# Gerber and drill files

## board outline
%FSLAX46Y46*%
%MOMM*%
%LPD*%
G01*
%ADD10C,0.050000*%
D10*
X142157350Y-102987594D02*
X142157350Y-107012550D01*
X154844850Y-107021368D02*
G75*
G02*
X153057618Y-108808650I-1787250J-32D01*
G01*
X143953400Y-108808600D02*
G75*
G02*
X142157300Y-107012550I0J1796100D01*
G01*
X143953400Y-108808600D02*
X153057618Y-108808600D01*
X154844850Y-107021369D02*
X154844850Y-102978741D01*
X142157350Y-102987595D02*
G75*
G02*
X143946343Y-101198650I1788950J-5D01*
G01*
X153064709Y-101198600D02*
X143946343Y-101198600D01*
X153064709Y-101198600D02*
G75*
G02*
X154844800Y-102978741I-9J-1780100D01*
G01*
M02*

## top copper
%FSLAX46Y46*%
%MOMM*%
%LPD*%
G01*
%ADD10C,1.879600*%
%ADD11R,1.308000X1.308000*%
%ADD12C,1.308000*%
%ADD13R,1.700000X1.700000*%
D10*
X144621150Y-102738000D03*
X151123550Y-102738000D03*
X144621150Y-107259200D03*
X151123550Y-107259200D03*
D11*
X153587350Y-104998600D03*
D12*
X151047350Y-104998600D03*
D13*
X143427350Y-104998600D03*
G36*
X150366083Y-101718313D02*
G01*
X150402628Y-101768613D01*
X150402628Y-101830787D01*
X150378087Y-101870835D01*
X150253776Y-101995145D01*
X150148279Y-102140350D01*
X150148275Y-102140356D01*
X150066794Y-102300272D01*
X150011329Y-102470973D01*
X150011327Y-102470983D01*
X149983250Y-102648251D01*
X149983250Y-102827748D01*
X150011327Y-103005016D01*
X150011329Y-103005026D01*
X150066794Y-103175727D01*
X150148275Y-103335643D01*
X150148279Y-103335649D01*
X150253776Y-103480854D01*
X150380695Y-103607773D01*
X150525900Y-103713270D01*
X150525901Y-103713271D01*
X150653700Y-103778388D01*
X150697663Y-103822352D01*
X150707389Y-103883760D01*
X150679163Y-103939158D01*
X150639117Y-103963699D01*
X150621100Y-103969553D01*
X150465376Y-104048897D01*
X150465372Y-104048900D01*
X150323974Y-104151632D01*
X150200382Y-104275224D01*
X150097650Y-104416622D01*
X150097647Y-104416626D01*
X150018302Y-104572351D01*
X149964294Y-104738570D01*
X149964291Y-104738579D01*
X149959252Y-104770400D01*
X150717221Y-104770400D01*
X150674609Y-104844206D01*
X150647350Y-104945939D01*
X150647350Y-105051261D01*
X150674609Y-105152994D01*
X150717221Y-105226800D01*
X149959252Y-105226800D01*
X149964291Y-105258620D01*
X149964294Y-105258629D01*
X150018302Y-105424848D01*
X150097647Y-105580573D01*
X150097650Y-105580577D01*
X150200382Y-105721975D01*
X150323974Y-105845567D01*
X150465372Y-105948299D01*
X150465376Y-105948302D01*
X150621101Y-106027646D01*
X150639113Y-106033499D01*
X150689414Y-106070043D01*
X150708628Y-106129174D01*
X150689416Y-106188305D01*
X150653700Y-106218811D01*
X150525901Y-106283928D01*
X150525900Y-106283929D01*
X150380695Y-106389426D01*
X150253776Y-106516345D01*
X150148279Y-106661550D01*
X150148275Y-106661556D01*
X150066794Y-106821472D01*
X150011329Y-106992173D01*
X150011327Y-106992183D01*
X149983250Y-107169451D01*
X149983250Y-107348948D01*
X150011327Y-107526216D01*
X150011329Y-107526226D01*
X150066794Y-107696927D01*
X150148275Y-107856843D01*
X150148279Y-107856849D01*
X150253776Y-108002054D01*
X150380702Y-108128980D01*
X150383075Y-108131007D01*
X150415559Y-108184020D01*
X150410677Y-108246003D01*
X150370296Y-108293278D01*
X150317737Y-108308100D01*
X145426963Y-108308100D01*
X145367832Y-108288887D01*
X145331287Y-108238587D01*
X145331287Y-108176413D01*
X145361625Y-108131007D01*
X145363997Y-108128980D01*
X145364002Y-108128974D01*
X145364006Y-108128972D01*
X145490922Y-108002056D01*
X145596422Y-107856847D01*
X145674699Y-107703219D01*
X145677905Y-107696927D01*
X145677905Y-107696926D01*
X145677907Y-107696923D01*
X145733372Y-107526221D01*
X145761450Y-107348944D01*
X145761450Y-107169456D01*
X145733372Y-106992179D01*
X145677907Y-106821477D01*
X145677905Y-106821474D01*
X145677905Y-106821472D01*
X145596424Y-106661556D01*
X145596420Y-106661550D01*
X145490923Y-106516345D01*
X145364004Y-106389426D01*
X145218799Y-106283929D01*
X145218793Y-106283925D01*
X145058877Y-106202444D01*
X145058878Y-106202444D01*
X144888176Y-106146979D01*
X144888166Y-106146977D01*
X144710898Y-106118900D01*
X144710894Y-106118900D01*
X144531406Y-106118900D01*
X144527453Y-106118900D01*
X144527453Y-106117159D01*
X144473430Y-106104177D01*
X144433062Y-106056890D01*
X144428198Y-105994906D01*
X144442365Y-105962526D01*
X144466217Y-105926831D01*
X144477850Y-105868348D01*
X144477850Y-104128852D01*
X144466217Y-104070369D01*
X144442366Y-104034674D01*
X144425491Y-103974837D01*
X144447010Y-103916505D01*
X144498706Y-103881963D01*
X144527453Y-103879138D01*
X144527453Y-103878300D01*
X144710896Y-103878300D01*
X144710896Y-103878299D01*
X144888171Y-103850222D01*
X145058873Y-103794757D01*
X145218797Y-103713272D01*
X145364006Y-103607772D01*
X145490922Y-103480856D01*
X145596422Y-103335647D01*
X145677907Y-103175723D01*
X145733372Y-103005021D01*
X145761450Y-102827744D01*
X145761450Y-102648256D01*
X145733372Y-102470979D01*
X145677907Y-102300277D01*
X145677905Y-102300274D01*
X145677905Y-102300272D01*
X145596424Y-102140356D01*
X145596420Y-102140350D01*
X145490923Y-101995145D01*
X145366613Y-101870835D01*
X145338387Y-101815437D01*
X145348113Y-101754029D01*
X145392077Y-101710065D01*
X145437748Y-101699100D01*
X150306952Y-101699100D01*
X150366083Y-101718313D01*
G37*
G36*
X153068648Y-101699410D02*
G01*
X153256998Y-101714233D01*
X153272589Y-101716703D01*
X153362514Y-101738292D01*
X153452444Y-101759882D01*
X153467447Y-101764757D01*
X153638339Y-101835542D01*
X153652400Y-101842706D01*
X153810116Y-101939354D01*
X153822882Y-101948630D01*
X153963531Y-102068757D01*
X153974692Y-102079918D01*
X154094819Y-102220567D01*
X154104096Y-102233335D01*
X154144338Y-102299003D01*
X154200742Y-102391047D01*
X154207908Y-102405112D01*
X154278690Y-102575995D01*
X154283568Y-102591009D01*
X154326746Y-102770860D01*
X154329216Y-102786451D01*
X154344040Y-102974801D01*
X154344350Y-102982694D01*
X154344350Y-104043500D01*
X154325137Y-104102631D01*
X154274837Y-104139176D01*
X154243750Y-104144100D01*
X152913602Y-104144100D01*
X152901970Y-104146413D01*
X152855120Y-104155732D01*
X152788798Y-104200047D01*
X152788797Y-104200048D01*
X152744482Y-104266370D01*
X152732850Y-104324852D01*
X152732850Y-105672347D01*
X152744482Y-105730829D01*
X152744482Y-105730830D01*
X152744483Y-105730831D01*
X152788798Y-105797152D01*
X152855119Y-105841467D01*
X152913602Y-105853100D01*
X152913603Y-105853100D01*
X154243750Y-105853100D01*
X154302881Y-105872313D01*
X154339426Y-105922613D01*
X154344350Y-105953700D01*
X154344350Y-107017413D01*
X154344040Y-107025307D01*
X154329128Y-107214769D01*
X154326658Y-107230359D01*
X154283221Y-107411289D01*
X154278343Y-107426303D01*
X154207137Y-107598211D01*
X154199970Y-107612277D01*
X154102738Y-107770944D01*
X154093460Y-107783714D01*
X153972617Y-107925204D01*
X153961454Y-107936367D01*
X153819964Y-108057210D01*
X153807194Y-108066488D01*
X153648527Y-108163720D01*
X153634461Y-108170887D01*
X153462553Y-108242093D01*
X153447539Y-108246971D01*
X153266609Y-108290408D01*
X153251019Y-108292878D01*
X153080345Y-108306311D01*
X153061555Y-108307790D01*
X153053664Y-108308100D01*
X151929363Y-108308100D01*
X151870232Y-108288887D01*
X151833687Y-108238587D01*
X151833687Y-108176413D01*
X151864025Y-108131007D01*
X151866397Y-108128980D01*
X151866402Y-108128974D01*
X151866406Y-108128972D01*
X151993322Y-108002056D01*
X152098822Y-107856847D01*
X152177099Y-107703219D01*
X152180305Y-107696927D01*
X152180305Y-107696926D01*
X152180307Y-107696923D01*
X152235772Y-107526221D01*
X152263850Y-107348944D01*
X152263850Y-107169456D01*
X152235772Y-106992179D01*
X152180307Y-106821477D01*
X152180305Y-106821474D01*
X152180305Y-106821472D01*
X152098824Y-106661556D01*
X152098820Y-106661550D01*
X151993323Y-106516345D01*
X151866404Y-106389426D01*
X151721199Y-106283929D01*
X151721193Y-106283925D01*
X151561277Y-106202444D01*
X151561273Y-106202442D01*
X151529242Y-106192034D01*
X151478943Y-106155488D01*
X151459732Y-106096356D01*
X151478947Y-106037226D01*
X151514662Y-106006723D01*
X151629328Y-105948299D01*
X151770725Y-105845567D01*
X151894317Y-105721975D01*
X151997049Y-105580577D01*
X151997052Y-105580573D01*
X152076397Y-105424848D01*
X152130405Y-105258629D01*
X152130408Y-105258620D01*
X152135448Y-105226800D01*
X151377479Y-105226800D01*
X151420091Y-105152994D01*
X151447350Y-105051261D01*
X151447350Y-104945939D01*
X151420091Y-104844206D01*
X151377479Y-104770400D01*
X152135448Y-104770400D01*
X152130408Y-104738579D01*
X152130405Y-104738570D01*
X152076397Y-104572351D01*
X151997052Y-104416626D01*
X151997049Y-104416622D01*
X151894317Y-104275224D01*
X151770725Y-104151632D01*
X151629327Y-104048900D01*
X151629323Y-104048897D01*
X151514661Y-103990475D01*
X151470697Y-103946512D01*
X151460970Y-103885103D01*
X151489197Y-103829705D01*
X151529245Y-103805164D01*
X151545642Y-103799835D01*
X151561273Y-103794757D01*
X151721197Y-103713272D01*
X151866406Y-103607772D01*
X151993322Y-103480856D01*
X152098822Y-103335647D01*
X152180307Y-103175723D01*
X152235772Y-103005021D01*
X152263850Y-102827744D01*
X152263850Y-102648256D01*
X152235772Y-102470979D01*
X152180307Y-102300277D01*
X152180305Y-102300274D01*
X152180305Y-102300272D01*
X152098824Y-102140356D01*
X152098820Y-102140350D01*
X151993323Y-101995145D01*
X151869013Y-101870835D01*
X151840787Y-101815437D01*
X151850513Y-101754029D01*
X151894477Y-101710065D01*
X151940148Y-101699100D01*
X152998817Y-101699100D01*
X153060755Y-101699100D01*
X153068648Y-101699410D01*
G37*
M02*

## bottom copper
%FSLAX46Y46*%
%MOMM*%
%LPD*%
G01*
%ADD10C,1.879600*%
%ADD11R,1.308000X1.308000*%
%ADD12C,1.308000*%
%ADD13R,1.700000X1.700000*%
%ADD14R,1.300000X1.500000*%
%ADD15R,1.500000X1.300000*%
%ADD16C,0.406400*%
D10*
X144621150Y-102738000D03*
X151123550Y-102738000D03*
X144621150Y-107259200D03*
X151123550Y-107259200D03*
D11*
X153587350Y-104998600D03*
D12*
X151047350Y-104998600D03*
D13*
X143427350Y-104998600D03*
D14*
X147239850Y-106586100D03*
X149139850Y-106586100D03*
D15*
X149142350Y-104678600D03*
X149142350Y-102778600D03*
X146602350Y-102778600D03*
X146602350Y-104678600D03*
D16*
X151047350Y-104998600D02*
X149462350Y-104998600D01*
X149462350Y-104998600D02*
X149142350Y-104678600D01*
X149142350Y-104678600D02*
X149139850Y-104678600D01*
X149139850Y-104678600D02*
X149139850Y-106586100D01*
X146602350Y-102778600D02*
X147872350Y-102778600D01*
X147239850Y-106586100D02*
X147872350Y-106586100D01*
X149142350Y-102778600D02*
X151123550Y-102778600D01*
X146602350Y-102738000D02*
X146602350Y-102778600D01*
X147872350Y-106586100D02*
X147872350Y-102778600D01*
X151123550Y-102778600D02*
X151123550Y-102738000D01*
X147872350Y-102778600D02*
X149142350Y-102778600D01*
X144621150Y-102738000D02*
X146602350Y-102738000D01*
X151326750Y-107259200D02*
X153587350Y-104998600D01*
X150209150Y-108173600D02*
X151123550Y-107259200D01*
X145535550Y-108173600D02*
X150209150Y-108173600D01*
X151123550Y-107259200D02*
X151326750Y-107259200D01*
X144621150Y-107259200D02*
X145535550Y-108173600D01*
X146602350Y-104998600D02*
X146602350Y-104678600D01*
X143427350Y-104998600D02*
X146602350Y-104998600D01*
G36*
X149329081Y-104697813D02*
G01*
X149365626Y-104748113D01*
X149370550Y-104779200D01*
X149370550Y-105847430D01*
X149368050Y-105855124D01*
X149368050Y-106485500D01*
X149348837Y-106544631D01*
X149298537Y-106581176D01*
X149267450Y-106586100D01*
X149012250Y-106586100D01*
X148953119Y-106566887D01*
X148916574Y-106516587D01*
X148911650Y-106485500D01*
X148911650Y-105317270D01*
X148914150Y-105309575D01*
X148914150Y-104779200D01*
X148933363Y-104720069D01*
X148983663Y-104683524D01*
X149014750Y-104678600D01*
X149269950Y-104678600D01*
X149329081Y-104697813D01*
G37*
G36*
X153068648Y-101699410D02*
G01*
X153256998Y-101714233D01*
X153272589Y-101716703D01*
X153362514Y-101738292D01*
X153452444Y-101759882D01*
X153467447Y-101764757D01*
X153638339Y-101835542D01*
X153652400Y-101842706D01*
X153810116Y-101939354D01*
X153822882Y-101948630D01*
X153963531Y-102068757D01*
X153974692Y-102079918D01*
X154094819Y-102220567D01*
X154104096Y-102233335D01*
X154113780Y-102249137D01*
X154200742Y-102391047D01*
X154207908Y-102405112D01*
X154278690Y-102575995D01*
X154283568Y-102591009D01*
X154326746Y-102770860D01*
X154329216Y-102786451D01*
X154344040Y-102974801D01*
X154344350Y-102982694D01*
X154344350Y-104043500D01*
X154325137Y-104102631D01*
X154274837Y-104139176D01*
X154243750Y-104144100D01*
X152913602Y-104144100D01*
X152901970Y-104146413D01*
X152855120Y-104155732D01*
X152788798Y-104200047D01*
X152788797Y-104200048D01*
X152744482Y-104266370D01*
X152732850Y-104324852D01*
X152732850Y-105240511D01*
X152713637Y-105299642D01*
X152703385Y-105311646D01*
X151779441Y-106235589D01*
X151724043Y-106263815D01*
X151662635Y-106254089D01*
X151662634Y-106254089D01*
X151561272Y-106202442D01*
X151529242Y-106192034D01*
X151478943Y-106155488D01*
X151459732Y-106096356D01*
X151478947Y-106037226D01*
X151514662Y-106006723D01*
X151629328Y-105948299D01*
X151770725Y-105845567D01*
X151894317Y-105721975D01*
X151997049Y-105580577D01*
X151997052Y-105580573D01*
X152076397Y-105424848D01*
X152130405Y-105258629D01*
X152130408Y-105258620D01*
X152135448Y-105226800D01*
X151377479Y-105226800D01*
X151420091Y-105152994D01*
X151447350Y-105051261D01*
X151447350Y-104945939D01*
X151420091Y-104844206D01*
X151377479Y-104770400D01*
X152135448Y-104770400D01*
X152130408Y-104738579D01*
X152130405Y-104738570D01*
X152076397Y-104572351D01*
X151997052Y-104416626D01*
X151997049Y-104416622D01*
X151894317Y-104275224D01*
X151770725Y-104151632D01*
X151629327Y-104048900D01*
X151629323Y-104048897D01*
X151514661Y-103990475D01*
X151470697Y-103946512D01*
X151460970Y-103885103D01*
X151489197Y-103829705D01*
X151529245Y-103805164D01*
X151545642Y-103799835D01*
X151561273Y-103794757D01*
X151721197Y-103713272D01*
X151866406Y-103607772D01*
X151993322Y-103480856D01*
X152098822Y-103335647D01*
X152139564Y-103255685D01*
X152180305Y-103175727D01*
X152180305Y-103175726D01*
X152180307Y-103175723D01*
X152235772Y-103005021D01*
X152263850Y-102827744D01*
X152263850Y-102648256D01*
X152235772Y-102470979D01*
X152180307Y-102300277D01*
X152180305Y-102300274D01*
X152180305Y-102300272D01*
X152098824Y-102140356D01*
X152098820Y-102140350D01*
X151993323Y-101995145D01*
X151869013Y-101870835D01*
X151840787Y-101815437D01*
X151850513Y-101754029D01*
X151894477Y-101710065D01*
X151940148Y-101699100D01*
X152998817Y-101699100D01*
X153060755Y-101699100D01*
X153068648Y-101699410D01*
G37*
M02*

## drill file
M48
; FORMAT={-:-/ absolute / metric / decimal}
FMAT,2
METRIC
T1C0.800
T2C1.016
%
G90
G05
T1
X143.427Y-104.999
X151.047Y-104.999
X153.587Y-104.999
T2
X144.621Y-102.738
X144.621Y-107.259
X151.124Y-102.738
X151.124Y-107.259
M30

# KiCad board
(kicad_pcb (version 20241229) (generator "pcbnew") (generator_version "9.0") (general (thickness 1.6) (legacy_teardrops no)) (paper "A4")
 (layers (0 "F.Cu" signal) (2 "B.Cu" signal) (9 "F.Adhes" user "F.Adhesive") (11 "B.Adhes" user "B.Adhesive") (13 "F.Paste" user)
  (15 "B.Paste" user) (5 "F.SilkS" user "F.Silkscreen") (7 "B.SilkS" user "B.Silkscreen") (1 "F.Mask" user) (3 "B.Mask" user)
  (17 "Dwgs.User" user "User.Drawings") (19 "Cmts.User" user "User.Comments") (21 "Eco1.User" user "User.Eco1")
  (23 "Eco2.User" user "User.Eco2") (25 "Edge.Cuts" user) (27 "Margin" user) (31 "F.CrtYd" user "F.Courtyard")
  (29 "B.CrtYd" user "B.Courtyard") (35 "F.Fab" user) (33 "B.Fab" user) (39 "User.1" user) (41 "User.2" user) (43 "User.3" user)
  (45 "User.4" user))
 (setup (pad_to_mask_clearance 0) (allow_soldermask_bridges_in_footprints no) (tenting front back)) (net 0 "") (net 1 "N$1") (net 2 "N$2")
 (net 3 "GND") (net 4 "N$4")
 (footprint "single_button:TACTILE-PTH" (layer "F.Cu") (at 147.87235 104.9986)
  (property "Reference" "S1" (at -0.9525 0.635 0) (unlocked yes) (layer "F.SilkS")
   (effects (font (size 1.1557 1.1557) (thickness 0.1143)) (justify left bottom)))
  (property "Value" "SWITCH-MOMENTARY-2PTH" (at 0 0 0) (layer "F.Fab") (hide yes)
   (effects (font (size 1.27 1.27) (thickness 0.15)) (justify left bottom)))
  (pad "1" thru_hole circle (at -3.2512 -2.2606) (size 1.8796 1.8796) (drill 1.016) (layers "*.Cu" "*.Mask") (remove_unused_layers no)
   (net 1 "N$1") (solder_mask_margin 0.0508) (thermal_bridge_angle 0))
  (pad "2" thru_hole circle (at 3.2512 -2.2606) (size 1.8796 1.8796) (drill 1.016) (layers "*.Cu" "*.Mask") (remove_unused_layers no)
   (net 1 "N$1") (solder_mask_margin 0.0508) (thermal_bridge_angle 0))
  (pad "3" thru_hole circle (at -3.2512 2.2606) (size 1.8796 1.8796) (drill 1.016) (layers "*.Cu" "*.Mask") (remove_unused_layers no)
   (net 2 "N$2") (solder_mask_margin 0.0508) (thermal_bridge_angle 0))
  (pad "4" thru_hole circle (at 3.2512 2.2606) (size 1.8796 1.8796) (drill 1.016) (layers "*.Cu" "*.Mask") (remove_unused_layers no)
   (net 2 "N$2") (solder_mask_margin 0.0508) (thermal_bridge_angle 0)))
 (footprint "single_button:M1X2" (layer "F.Cu") (at 152.31735 104.9986 180)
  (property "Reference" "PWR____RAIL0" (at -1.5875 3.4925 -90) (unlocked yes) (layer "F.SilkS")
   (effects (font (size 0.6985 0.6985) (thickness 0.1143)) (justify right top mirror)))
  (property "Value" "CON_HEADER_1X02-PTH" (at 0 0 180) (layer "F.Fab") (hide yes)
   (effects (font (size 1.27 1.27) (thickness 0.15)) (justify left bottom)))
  (pad "1" thru_hole rect (at -1.27 0 180) (size 1.308 1.308) (drill 0.8) (layers "*.Cu" "*.Mask") (remove_unused_layers no) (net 2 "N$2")
   (solder_mask_margin 0.0508) (thermal_bridge_angle 0))
  (pad "2" thru_hole circle (at 1.27 0 180) (size 1.308 1.308) (drill 0.8) (layers "*.Cu" "*.Mask") (remove_unused_layers no) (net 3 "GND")
   (solder_mask_margin 0.0508) (thermal_bridge_angle 0)))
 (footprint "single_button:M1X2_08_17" (layer "F.Cu") (at 143.42735 104.9986)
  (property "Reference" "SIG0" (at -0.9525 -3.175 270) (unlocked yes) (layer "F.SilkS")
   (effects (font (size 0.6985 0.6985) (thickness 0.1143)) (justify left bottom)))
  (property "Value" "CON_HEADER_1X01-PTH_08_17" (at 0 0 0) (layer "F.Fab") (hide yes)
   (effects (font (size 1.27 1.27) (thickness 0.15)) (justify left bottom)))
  (pad "1" thru_hole rect (at 0 0) (size 1.7 1.7) (drill 0.8) (layers "*.Cu" "*.Mask") (remove_unused_layers no) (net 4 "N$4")
   (solder_mask_margin 0.0508) (thermal_bridge_angle 0)))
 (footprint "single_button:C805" (layer "B.Cu") (at 148.18985 106.5861)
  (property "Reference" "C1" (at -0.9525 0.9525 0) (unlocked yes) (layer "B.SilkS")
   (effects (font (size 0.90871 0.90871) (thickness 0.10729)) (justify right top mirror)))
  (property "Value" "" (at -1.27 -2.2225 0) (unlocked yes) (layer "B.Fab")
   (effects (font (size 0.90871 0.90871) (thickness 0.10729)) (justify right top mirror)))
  (pad "1" smd rect (at -0.95 0) (size 1.3 1.5) (layers "B.Cu" "B.Mask" "B.Paste") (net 1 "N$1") (solder_mask_margin 0.0508)
   (solder_paste_margin 0) (thermal_bridge_angle 0))
  (pad "2" smd rect (at 0.95 0) (size 1.3 1.5) (layers "B.Cu" "B.Mask" "B.Paste") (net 3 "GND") (solder_mask_margin 0.0508)
   (solder_paste_margin 0) (thermal_bridge_angle 0)))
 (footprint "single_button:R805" (layer "B.Cu") (at 149.14235 103.7286 90)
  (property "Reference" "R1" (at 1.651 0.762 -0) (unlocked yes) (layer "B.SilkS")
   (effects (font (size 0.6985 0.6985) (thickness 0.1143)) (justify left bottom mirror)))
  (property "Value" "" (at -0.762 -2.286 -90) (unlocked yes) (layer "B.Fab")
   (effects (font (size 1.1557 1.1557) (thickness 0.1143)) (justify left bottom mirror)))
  (pad "1" smd rect (at -0.95 0 90) (size 1.3 1.5) (layers "B.Cu" "B.Mask" "B.Paste") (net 3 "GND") (solder_mask_margin 0.0508)
   (solder_paste_margin 0) (thermal_bridge_angle 0))
  (pad "2" smd rect (at 0.95 0 90) (size 1.3 1.5) (layers "B.Cu" "B.Mask" "B.Paste") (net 1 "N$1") (solder_mask_margin 0.0508)
   (solder_paste_margin 0) (thermal_bridge_angle 0)))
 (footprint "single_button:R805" (layer "B.Cu") (at 146.60235 103.7286 -90)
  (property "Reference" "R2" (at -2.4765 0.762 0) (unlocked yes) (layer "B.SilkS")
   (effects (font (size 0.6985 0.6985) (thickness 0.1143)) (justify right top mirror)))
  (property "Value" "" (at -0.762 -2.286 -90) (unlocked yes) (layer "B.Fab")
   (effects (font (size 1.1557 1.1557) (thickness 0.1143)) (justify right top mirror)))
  (pad "1" smd rect (at -0.95 0 270) (size 1.3 1.5) (layers "B.Cu" "B.Mask" "B.Paste") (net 1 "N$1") (solder_mask_margin 0.0508)
   (solder_paste_margin 0) (thermal_bridge_angle 0))
  (pad "2" smd rect (at 0.95 0 270) (size 1.3 1.5) (layers "B.Cu" "B.Mask" "B.Paste") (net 4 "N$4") (solder_mask_margin 0.0508)
   (solder_paste_margin 0) (thermal_bridge_angle 0)))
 (gr_line (start 142.15735 102.987594) (end 142.15735 107.01255) (stroke (width 0.05) (type solid)) (layer "Edge.Cuts"))
 (gr_arc (start 154.84485 107.021368) (mid 154.321382 108.285132) (end 153.057618 108.8086) (stroke (width 0.05) (type solid))
  (layer "Edge.Cuts"))
 (gr_arc (start 143.9534 108.8086) (mid 142.683401 108.282549) (end 142.15735 107.01255) (stroke (width 0.05) (type solid))
  (layer "Edge.Cuts"))
 (gr_line (start 143.9534 108.8086) (end 153.057618 108.8086) (stroke (width 0.05) (type solid)) (layer "Edge.Cuts"))
 (gr_line (start 154.84485 107.021369) (end 154.84485 102.978741) (stroke (width 0.05) (type solid)) (layer "Edge.Cuts"))
 (gr_arc (start 142.15735 102.987595) (mid 142.681334 101.722585) (end 143.946343 101.1986) (stroke (width 0.05) (type solid))
  (layer "Edge.Cuts"))
 (gr_line (start 153.064709 101.1986) (end 143.946343 101.1986) (stroke (width 0.05) (type solid)) (layer "Edge.Cuts"))
 (gr_arc (start 153.064709 101.1986) (mid 154.323459 101.719991) (end 154.84485 102.978741) (stroke (width 0.05) (type solid))
  (layer "Edge.Cuts"))
 (segment (start 151.04735 104.9986) (end 149.46235 104.9986) (width 0.4064) (layer "B.Cu") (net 3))
 (segment (start 149.46235 104.9986) (end 149.14235 104.6786) (width 0.4064) (layer "B.Cu") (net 3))
 (segment (start 149.14235 104.6786) (end 149.13985 104.6786) (width 0.4064) (layer "B.Cu") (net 3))
 (segment (start 149.13985 104.6786) (end 149.13985 106.5861) (width 0.4064) (layer "B.Cu") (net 3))
 (segment (start 146.60235 102.7786) (end 147.87235 102.7786) (width 0.4064) (layer "B.Cu") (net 1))
 (segment (start 147.23985 106.5861) (end 147.87235 106.5861) (width 0.4064) (layer "B.Cu") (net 1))
 (segment (start 149.14235 102.7786) (end 151.12355 102.7786) (width 0.4064) (layer "B.Cu") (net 1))
 (segment (start 146.60235 102.738) (end 146.60235 102.7786) (width 0.4064) (layer "B.Cu") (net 1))
 (segment (start 147.87235 106.5861) (end 147.87235 102.7786) (width 0.4064) (layer "B.Cu") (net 1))
 (segment (start 151.12355 102.7786) (end 151.12355 102.738) (width 0.4064) (layer "B.Cu") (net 1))
 (segment (start 147.87235 102.7786) (end 149.14235 102.7786) (width 0.4064) (layer "B.Cu") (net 1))
 (segment (start 144.62115 102.738) (end 146.60235 102.738) (width 0.4064) (layer "B.Cu") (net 1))
 (segment (start 151.32675 107.2592) (end 153.58735 104.9986) (width 0.4064) (layer "B.Cu") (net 2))
 (segment (start 150.20915 108.1736) (end 151.12355 107.2592) (width 0.4064) (layer "B.Cu") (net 2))
 (segment (start 145.53555 108.1736) (end 150.20915 108.1736) (width 0.4064) (layer "B.Cu") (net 2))
 (segment (start 151.12355 107.2592) (end 151.32675 107.2592) (width 0.4064) (layer "B.Cu") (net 2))
 (segment (start 144.62115 107.2592) (end 145.53555 108.1736) (width 0.4064) (layer "B.Cu") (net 2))
 (segment (start 146.60235 104.9986) (end 146.60235 104.6786) (width 0.4064) (layer "B.Cu") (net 4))
 (segment (start 143.42735 104.9986) (end 146.60235 104.9986) (width 0.4064) (layer "B.Cu") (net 4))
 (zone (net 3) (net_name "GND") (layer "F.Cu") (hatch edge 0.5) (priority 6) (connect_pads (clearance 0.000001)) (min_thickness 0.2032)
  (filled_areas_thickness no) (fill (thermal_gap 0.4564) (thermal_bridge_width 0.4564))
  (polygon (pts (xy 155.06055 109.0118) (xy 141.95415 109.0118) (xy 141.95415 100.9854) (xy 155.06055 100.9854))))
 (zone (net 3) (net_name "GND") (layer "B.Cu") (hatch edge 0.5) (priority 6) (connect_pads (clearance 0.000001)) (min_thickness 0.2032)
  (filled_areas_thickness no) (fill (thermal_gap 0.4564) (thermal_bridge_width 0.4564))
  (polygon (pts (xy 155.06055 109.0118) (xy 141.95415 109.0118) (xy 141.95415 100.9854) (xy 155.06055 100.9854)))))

